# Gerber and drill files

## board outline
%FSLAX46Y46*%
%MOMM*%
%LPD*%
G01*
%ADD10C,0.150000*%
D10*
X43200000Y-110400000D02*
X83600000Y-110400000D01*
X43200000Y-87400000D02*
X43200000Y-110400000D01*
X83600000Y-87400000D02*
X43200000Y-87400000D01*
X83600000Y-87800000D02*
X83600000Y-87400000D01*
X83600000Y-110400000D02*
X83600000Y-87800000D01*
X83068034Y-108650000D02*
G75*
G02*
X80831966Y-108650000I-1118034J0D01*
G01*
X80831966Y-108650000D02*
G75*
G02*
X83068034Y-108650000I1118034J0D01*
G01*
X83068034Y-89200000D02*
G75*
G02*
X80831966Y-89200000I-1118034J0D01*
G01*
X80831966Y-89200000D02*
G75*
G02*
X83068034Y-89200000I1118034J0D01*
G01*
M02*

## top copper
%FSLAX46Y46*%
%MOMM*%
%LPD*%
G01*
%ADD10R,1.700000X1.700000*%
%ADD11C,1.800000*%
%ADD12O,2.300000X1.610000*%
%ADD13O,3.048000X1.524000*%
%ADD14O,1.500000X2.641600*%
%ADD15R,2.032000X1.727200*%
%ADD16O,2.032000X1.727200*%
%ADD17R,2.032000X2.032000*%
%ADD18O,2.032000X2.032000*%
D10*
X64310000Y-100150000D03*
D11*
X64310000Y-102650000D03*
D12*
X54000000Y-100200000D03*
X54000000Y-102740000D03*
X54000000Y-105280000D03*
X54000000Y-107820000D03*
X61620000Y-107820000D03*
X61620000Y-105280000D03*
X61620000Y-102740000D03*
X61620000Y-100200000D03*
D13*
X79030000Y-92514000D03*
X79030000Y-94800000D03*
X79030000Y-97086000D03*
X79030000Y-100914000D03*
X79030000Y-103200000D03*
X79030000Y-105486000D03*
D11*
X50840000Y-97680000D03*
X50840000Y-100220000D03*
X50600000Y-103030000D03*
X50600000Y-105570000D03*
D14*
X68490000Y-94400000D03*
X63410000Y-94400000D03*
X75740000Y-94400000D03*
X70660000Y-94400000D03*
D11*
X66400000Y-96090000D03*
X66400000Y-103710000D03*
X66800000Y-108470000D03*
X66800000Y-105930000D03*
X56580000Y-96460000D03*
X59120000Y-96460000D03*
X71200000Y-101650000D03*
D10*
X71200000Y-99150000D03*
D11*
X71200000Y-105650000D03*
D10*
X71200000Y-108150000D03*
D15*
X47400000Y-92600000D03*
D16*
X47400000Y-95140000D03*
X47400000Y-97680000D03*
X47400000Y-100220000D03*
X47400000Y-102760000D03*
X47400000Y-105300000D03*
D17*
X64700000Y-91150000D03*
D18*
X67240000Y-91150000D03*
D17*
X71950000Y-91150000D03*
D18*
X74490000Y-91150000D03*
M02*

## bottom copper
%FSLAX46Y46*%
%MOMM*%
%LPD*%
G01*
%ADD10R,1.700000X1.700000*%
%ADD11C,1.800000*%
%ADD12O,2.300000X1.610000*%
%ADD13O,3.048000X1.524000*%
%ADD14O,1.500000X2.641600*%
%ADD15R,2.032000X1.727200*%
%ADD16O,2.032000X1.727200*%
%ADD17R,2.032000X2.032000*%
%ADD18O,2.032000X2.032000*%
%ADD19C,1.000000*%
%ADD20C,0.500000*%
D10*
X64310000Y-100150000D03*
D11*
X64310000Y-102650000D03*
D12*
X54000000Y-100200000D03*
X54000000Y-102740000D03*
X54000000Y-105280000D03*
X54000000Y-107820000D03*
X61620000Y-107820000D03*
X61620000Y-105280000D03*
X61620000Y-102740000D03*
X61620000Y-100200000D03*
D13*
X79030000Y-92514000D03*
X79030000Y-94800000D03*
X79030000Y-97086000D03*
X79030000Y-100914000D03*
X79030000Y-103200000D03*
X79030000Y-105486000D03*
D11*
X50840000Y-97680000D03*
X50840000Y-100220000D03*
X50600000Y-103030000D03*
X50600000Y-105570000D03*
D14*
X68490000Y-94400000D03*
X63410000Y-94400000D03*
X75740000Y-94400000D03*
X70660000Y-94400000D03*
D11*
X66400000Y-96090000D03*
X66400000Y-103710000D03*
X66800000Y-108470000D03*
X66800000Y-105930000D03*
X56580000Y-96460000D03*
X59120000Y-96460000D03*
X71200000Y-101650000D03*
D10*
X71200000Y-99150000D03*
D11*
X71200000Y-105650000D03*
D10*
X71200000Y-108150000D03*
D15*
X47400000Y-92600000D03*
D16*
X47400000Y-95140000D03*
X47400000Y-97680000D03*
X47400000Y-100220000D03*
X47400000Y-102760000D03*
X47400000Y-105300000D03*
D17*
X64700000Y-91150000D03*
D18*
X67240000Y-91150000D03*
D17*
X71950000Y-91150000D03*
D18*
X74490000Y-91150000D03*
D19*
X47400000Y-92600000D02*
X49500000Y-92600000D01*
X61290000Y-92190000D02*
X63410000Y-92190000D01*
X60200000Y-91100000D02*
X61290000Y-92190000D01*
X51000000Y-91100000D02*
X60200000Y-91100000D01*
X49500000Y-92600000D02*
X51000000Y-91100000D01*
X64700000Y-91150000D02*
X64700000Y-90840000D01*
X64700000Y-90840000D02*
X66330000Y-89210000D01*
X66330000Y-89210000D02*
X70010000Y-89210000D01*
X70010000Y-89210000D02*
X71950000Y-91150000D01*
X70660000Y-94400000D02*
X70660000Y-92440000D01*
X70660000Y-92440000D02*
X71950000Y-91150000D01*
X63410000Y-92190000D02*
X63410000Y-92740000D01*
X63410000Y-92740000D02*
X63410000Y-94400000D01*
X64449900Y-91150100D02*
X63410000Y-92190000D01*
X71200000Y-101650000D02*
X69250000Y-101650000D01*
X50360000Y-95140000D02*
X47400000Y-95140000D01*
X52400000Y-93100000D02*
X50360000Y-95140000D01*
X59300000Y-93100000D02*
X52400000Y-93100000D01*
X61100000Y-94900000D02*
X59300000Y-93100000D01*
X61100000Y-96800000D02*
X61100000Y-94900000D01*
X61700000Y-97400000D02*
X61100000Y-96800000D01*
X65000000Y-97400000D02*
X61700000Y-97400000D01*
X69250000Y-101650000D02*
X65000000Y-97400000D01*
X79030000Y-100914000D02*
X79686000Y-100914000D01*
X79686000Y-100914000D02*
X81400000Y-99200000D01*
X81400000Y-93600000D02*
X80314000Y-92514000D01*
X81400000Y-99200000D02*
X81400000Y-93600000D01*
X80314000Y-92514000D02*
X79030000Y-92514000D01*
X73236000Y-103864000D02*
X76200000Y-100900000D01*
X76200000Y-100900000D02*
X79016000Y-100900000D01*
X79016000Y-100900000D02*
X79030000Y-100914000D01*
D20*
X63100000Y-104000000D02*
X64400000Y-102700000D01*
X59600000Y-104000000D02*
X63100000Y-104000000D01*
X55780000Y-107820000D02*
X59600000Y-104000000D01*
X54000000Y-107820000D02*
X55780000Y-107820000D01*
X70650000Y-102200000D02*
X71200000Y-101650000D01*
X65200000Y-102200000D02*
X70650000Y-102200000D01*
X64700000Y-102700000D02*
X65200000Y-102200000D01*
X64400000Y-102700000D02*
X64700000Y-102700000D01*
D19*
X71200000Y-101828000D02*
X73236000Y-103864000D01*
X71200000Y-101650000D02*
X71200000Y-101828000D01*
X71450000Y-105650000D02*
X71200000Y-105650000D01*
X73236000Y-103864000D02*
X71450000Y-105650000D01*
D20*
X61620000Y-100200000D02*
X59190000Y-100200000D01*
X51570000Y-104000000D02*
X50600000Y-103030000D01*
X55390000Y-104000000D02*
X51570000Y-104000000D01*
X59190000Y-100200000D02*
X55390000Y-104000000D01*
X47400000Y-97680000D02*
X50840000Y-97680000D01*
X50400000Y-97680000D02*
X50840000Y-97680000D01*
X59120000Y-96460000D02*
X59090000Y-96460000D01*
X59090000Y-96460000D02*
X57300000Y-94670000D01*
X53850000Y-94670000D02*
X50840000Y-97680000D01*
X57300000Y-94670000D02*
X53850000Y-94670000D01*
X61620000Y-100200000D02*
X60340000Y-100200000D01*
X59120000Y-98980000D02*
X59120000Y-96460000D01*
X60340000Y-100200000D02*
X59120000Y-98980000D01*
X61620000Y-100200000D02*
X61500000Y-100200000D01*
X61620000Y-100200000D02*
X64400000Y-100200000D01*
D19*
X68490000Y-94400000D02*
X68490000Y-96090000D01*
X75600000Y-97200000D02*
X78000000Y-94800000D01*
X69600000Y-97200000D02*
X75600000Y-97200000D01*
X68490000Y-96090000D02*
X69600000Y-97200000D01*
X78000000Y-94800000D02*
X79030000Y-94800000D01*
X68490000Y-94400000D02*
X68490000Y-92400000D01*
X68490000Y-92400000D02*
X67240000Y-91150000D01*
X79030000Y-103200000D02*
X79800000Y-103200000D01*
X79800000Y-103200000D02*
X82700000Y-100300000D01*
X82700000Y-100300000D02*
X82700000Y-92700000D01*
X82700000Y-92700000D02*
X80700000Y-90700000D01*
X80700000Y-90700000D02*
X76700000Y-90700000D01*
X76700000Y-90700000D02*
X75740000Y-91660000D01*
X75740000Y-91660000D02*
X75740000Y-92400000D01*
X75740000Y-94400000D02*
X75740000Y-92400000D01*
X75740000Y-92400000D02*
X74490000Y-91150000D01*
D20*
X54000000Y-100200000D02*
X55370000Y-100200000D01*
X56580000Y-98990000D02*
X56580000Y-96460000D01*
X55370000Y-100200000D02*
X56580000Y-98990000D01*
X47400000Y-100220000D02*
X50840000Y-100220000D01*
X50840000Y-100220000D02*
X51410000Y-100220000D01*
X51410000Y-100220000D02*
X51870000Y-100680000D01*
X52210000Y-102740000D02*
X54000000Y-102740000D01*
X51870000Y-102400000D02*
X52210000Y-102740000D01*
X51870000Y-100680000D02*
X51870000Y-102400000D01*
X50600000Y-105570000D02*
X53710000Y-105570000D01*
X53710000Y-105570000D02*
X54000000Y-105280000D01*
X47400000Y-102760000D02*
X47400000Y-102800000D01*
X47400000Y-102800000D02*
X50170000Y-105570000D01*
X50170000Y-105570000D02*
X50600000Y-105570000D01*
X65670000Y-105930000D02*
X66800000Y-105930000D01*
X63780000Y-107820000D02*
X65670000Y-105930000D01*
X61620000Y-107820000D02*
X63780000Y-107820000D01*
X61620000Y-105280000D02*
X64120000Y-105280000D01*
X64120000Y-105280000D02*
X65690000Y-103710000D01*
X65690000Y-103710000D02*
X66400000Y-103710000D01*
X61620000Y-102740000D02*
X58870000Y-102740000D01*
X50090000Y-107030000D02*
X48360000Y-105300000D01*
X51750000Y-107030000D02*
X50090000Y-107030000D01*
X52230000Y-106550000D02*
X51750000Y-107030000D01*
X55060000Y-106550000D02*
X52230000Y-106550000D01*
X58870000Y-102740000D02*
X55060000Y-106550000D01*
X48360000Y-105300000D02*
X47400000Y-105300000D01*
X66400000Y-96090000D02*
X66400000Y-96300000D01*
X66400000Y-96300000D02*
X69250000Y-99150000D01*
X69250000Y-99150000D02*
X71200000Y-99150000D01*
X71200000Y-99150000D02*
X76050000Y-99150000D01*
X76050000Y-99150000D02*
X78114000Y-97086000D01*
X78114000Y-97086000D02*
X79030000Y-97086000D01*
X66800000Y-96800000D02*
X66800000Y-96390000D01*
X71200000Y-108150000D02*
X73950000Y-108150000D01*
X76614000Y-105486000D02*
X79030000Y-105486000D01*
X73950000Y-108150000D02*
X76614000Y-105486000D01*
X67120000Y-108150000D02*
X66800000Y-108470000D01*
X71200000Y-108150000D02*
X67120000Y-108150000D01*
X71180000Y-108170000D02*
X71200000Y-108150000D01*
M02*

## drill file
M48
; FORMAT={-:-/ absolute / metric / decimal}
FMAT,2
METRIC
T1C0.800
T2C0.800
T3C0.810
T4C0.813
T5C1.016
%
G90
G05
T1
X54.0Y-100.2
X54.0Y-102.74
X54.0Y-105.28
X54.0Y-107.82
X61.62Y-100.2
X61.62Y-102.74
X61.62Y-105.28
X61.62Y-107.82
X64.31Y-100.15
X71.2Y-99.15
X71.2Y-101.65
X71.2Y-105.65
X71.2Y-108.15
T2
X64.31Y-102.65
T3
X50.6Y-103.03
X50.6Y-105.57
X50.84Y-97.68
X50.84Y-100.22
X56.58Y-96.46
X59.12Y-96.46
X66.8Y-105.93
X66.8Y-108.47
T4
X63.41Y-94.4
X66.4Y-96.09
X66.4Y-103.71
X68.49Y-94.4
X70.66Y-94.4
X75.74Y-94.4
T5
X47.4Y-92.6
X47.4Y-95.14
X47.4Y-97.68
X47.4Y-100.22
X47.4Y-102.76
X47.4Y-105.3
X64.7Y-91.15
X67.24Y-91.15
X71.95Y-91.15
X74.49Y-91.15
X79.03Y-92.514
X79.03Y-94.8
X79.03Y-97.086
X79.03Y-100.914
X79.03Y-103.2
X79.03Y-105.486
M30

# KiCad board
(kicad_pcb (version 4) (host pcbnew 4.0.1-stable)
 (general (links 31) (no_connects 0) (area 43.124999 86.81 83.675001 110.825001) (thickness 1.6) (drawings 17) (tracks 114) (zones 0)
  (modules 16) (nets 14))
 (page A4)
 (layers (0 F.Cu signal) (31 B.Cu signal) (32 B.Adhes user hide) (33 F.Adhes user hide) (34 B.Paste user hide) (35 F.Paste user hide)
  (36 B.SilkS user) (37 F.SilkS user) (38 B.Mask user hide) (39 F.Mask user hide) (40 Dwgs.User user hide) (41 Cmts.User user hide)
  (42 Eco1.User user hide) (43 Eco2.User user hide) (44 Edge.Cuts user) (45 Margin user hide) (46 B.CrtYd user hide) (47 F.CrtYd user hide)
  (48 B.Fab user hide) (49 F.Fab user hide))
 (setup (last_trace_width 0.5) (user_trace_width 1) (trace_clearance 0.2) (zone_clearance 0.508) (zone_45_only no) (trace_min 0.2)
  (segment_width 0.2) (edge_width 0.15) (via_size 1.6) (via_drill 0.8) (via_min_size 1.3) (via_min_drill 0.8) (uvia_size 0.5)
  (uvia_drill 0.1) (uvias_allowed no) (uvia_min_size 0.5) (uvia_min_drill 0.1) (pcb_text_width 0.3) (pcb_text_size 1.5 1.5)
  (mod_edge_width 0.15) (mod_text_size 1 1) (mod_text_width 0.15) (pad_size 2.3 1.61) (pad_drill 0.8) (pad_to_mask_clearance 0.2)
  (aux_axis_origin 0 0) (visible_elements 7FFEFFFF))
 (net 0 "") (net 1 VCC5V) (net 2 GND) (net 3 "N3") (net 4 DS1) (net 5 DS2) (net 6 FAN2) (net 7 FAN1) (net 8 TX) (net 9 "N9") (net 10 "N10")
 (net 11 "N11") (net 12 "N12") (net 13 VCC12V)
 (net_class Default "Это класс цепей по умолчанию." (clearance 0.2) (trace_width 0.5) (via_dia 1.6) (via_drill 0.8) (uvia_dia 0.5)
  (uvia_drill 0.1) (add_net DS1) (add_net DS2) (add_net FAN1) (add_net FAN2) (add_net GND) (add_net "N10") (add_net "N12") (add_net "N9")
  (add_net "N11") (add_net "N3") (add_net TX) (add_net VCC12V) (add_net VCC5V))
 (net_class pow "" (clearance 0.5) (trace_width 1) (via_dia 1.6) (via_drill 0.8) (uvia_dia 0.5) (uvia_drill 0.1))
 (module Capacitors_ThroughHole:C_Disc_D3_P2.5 (layer F.Cu) (at 64.31 100.15 270)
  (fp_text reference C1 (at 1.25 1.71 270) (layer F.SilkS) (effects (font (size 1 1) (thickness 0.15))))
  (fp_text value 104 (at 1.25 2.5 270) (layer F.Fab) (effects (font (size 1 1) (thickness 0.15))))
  (pad 1 thru_hole rect (at 0 0 270) (size 1.7 1.7) (drill 0.8) (layers *.Cu *.Mask F.SilkS) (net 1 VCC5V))
  (pad 2 thru_hole circle (at 2.5 0 270) (size 1.8 1.8) (drill 0.8001) (layers *.Cu *.Mask F.SilkS) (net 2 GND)))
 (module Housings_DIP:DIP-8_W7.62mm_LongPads (layer F.Cu) (at 54 100.2)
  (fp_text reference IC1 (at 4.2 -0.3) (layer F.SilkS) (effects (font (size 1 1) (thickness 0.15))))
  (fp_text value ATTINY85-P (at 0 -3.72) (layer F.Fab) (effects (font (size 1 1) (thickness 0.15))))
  (pad 1 thru_hole oval (at 0 0) (size 2.3 1.61) (drill 0.8) (layers *.Cu *.Mask F.SilkS) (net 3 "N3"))
  (pad 2 thru_hole oval (at 0 2.54) (size 2.3 1.61) (drill 0.8) (layers *.Cu *.Mask F.SilkS) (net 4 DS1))
  (pad 3 thru_hole oval (at 0 5.08) (size 2.3 1.61) (drill 0.8) (layers *.Cu *.Mask F.SilkS) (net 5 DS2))
  (pad 4 thru_hole oval (at 0 7.62) (size 2.3 1.61) (drill 0.8) (layers *.Cu *.Mask F.SilkS) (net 2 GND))
  (pad 5 thru_hole oval (at 7.62 7.62) (size 2.3 1.61) (drill 0.8) (layers *.Cu *.Mask F.SilkS) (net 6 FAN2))
  (pad 6 thru_hole oval (at 7.62 5.08) (size 2.3 1.61) (drill 0.8) (layers *.Cu *.Mask F.SilkS) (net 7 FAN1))
  (pad 7 thru_hole oval (at 7.62 2.54) (size 2.3 1.61) (drill 0.8) (layers *.Cu *.Mask F.SilkS) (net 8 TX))
  (pad 8 thru_hole oval (at 7.62 0) (size 2.3 1.61) (drill 0.8) (layers *.Cu *.Mask F.SilkS) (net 1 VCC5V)))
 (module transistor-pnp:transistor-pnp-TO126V (layer F.Cu) (at 80.3 94.8 270)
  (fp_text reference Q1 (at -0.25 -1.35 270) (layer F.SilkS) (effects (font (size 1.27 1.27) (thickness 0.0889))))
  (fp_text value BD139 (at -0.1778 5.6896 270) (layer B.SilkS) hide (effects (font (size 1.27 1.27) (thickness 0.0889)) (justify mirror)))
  (pad 1 thru_hole oval (at -2.286 1.27 270) (size 1.524 3.048) (drill 1.016) (layers *.Cu F.Paste F.SilkS F.Mask) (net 2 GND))
  (pad 2 thru_hole oval (at 0 1.27 270) (size 1.524 3.048) (drill 1.016) (layers *.Cu F.Paste F.SilkS F.Mask) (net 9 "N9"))
  (pad 3 thru_hole oval (at 2.286 1.27 270) (size 1.524 3.048) (drill 1.016) (layers *.Cu F.Paste F.SilkS F.Mask) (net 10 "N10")))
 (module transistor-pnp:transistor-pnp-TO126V (layer F.Cu) (at 80.3 103.2 270)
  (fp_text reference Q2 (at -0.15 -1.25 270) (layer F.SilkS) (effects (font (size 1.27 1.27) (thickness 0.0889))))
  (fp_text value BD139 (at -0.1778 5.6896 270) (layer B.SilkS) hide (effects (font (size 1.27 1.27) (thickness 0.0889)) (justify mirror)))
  (pad 1 thru_hole oval (at -2.286 1.27 270) (size 1.524 3.048) (drill 1.016) (layers *.Cu F.Paste F.SilkS F.Mask) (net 2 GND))
  (pad 2 thru_hole oval (at 0 1.27 270) (size 1.524 3.048) (drill 1.016) (layers *.Cu F.Paste F.SilkS F.Mask) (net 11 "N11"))
  (pad 3 thru_hole oval (at 2.286 1.27 270) (size 1.524 3.048) (drill 1.016) (layers *.Cu F.Paste F.SilkS F.Mask) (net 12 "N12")))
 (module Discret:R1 (layer F.Cu) (at 50.84 98.95 270)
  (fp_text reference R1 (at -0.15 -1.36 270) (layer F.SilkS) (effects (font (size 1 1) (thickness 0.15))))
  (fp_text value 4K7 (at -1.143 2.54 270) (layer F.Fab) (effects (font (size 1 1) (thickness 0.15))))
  (pad 1 thru_hole circle (at -1.27 0 270) (size 1.8 1.8) (drill 0.81) (layers *.Cu *.Mask F.SilkS) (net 1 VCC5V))
  (pad 2 thru_hole circle (at 1.27 0 270) (size 1.8 1.8) (drill 0.81) (layers *.Cu *.Mask F.SilkS) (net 4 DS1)))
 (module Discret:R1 (layer F.Cu) (at 50.6 104.3 270)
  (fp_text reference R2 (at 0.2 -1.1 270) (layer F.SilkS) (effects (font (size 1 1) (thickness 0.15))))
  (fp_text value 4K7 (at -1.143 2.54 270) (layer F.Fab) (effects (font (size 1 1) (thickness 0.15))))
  (pad 1 thru_hole circle (at -1.27 0 270) (size 1.8 1.8) (drill 0.81) (layers *.Cu *.Mask F.SilkS) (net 1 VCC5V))
  (pad 2 thru_hole circle (at 1.27 0 270) (size 1.8 1.8) (drill 0.81) (layers *.Cu *.Mask F.SilkS) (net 5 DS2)))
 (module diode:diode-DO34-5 (layer F.Cu) (at 65.95 94.4)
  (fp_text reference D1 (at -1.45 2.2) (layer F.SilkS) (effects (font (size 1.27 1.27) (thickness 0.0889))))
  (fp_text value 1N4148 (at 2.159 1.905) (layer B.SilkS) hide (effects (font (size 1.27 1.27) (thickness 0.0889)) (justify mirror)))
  (pad 2 thru_hole oval (at 2.54 0) (size 1.5 2.6416) (drill 0.8128) (layers *.Cu F.Paste F.SilkS F.Mask) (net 9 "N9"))
  (pad 1 thru_hole oval (at -2.54 0) (size 1.5 2.6416) (drill 0.8128) (layers *.Cu F.Paste F.SilkS F.Mask) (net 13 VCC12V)))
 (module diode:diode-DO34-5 (layer F.Cu) (at 73.2 94.4)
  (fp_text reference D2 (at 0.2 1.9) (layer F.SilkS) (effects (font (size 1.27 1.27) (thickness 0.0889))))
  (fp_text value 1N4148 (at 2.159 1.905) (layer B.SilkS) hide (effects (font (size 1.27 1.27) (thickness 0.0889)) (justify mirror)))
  (pad 2 thru_hole oval (at 2.54 0) (size 1.5 2.6416) (drill 0.8128) (layers *.Cu F.Paste F.SilkS F.Mask) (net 11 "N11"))
  (pad 1 thru_hole oval (at -2.54 0) (size 1.5 2.6416) (drill 0.8128) (layers *.Cu F.Paste F.SilkS F.Mask) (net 13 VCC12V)))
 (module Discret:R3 (layer F.Cu) (at 66.4 99.9 270)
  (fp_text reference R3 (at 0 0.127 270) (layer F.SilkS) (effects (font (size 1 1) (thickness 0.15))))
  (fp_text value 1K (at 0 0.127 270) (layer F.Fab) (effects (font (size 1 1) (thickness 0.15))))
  (pad 1 thru_hole circle (at -3.81 0 270) (size 1.8 1.8) (drill 0.8128) (layers *.Cu *.Mask F.SilkS) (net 10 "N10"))
  (pad 2 thru_hole circle (at 3.81 0 270) (size 1.8 1.8) (drill 0.8128) (layers *.Cu *.Mask F.SilkS) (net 7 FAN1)))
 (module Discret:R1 (layer F.Cu) (at 66.8 107.2 90)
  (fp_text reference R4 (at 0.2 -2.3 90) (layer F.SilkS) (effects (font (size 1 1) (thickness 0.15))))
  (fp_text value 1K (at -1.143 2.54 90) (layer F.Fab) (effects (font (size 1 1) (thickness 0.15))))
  (pad 1 thru_hole circle (at -1.27 0 90) (size 1.8 1.8) (drill 0.81) (layers *.Cu *.Mask F.SilkS) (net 12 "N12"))
  (pad 2 thru_hole circle (at 1.27 0 90) (size 1.8 1.8) (drill 0.81) (layers *.Cu *.Mask F.SilkS) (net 6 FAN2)))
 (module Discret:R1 (layer F.Cu) (at 57.85 96.46)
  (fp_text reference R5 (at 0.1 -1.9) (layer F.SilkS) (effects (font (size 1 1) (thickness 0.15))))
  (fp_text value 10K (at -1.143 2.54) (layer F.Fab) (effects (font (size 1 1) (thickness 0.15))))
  (pad 1 thru_hole circle (at -1.27 0) (size 1.8 1.8) (drill 0.81) (layers *.Cu *.Mask F.SilkS) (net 3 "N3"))
  (pad 2 thru_hole circle (at 1.27 0) (size 1.8 1.8) (drill 0.81) (layers *.Cu *.Mask F.SilkS) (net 1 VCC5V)))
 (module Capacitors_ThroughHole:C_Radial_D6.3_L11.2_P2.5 (layer F.Cu) (at 71.2 99.15 270)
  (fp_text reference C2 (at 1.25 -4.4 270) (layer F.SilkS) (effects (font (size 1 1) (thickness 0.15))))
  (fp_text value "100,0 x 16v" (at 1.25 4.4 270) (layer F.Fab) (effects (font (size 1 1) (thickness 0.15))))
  (pad 2 thru_hole circle (at 2.5 0 270) (size 1.8 1.8) (drill 0.8) (layers *.Cu *.Mask F.SilkS) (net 2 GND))
  (pad 1 thru_hole rect (at 0 0 270) (size 1.7 1.7) (drill 0.8) (layers *.Cu *.Mask F.SilkS) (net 10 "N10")))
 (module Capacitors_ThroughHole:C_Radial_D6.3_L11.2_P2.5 (layer F.Cu) (at 71.2 108.15 90)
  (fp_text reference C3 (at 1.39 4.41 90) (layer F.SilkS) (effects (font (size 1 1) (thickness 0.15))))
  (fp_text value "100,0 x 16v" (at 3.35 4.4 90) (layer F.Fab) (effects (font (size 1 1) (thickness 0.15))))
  (pad 2 thru_hole circle (at 2.5 0 90) (size 1.8 1.8) (drill 0.8) (layers *.Cu *.Mask F.SilkS) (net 2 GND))
  (pad 1 thru_hole rect (at 0 0 90) (size 1.7 1.7) (drill 0.8) (layers *.Cu *.Mask F.SilkS) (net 12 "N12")))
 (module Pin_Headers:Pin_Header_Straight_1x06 (layer F.Cu) (at 47.4 92.6)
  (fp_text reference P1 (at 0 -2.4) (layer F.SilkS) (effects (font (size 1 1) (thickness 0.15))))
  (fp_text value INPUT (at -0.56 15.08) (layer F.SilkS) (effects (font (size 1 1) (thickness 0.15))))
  (pad 1 thru_hole rect (at 0 0) (size 2.032 1.7272) (drill 1.016) (layers *.Cu *.Mask F.SilkS) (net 13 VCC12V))
  (pad 2 thru_hole oval (at 0 2.54) (size 2.032 1.7272) (drill 1.016) (layers *.Cu *.Mask F.SilkS) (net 2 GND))
  (pad 3 thru_hole oval (at 0 5.08) (size 2.032 1.7272) (drill 1.016) (layers *.Cu *.Mask F.SilkS) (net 1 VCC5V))
  (pad 4 thru_hole oval (at 0 7.62) (size 2.032 1.7272) (drill 1.016) (layers *.Cu *.Mask F.SilkS) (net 4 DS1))
  (pad 5 thru_hole oval (at 0 10.16) (size 2.032 1.7272) (drill 1.016) (layers *.Cu *.Mask F.SilkS) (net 5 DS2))
  (pad 6 thru_hole oval (at 0 12.7) (size 2.032 1.7272) (drill 1.016) (layers *.Cu *.Mask F.SilkS) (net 8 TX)))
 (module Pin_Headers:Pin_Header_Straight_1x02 (layer F.Cu) (at 64.7 91.15 90)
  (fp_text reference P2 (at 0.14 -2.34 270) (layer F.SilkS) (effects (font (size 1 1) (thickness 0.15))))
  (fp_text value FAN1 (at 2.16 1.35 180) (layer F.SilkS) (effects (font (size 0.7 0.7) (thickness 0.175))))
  (pad 1 thru_hole rect (at 0 0 90) (size 2.032 2.032) (drill 1.016) (layers *.Cu *.Mask F.SilkS) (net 13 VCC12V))
  (pad 2 thru_hole oval (at 0 2.54 90) (size 2.032 2.032) (drill 1.016) (layers *.Cu *.Mask F.SilkS) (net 9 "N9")))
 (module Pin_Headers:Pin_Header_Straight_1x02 (layer F.Cu) (at 71.95 91.15 90)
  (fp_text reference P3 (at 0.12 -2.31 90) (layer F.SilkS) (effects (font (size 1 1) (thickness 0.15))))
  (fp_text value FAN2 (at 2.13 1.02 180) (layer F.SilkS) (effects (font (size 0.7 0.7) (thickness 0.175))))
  (pad 1 thru_hole rect (at 0 0 90) (size 2.032 2.032) (drill 1.016) (layers *.Cu *.Mask F.SilkS) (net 13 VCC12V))
  (pad 2 thru_hole oval (at 0 2.54 90) (size 2.032 2.032) (drill 1.016) (layers *.Cu *.Mask F.SilkS) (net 11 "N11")))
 (gr_line (start 43.2 110.4) (end 83.6 110.4) (angle 90) (layer Edge.Cuts) (width 0.15))
 (gr_line (start 43.2 87.4) (end 43.2 110.4) (angle 90) (layer Edge.Cuts) (width 0.15))
 (gr_line (start 83.6 87.4) (end 43.2 87.4) (angle 90) (layer Edge.Cuts) (width 0.15))
 (gr_line (start 83.6 87.8) (end 83.6 87.4) (angle 90) (layer Edge.Cuts) (width 0.15))
 (gr_line (start 83.6 110.4) (end 83.6 87.8) (angle 90) (layer Edge.Cuts) (width 0.15))
 (gr_circle (center 81.95 108.65) (end 82.95 108.15) (layer Edge.Cuts) (width 0.15))
 (gr_circle (center 81.95 89.2) (end 82.95 88.7) (layer Edge.Cuts) (width 0.15))
 (segment (start 47.4 92.6) (end 49.5 92.6) (width 1) (layer B.Cu) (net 13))
 (segment (start 61.29 92.19) (end 63.41 92.19) (width 1) (layer B.Cu) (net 13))
 (segment (start 60.2 91.1) (end 61.29 92.19) (width 1) (layer B.Cu) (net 13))
 (segment (start 51 91.1) (end 60.2 91.1) (width 1) (layer B.Cu) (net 13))
 (segment (start 49.5 92.6) (end 51 91.1) (width 1) (layer B.Cu) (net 13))
 (segment (start 64.7 91.15) (end 64.7 90.84) (width 1) (layer B.Cu) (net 13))
 (segment (start 64.7 90.84) (end 66.33 89.21) (width 1) (layer B.Cu) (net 13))
 (segment (start 66.33 89.21) (end 70.01 89.21) (width 1) (layer B.Cu) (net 13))
 (segment (start 70.01 89.21) (end 71.95 91.15) (width 1) (layer B.Cu) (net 13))
 (segment (start 70.66 94.4) (end 70.66 92.44) (width 1) (layer B.Cu) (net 13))
 (segment (start 70.66 92.44) (end 71.95 91.15) (width 1) (layer B.Cu) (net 13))
 (segment (start 63.41 92.19) (end 63.41 92.74) (width 1) (layer B.Cu) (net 13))
 (segment (start 63.41 92.74) (end 63.41 94.4) (width 1) (layer B.Cu) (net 13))
 (segment (start 64.4499 91.1501) (end 63.41 92.19) (width 1) (layer B.Cu) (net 13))
 (segment (start 71.2 101.65) (end 69.25 101.65) (width 1) (layer B.Cu) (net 2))
 (segment (start 50.36 95.14) (end 47.4 95.14) (width 1) (layer B.Cu) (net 2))
 (segment (start 52.4 93.1) (end 50.36 95.14) (width 1) (layer B.Cu) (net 2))
 (segment (start 59.3 93.1) (end 52.4 93.1) (width 1) (layer B.Cu) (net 2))
 (segment (start 61.1 94.9) (end 59.3 93.1) (width 1) (layer B.Cu) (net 2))
 (segment (start 61.1 96.8) (end 61.1 94.9) (width 1) (layer B.Cu) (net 2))
 (segment (start 61.7 97.4) (end 61.1 96.8) (width 1) (layer B.Cu) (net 2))
 (segment (start 65 97.4) (end 61.7 97.4) (width 1) (layer B.Cu) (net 2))
 (segment (start 69.25 101.65) (end 65 97.4) (width 1) (layer B.Cu) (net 2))
 (segment (start 79.03 100.914) (end 79.686 100.914) (width 1) (layer B.Cu) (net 2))
 (segment (start 79.686 100.914) (end 81.4 99.2) (width 1) (layer B.Cu) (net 2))
 (segment (start 81.4 93.6) (end 80.314 92.514) (width 1) (layer B.Cu) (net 2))
 (segment (start 81.4 99.2) (end 81.4 93.6) (width 1) (layer B.Cu) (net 2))
 (segment (start 80.314 92.514) (end 79.03 92.514) (width 1) (layer B.Cu) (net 2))
 (segment (start 73.236 103.864) (end 76.2 100.9) (width 1) (layer B.Cu) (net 2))
 (segment (start 76.2 100.9) (end 79.016 100.9) (width 1) (layer B.Cu) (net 2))
 (segment (start 79.016 100.9) (end 79.03 100.914) (width 1) (layer B.Cu) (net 2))
 (segment (start 63.1 104) (end 64.4 102.7) (width 0.5) (layer B.Cu) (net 2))
 (segment (start 59.6 104) (end 63.1 104) (width 0.5) (layer B.Cu) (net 2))
 (segment (start 55.78 107.82) (end 59.6 104) (width 0.5) (layer B.Cu) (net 2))
 (segment (start 54 107.82) (end 55.78 107.82) (width 0.5) (layer B.Cu) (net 2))
 (segment (start 70.65 102.2) (end 71.2 101.65) (width 0.5) (layer B.Cu) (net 2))
 (segment (start 65.2 102.2) (end 70.65 102.2) (width 0.5) (layer B.Cu) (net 2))
 (segment (start 64.7 102.7) (end 65.2 102.2) (width 0.5) (layer B.Cu) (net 2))
 (segment (start 64.4 102.7) (end 64.7 102.7) (width 0.5) (layer B.Cu) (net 2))
 (segment (start 71.2 101.828) (end 73.236 103.864) (width 1) (layer B.Cu) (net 2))
 (segment (start 71.2 101.65) (end 71.2 101.828) (width 1) (layer B.Cu) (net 2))
 (segment (start 71.45 105.65) (end 71.2 105.65) (width 1) (layer B.Cu) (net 2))
 (segment (start 73.236 103.864) (end 71.45 105.65) (width 1) (layer B.Cu) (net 2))
 (segment (start 61.62 100.2) (end 59.19 100.2) (width 0.5) (layer B.Cu) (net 1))
 (segment (start 51.57 104) (end 50.6 103.03) (width 0.5) (layer B.Cu) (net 1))
 (segment (start 55.39 104) (end 51.57 104) (width 0.5) (layer B.Cu) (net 1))
 (segment (start 59.19 100.2) (end 55.39 104) (width 0.5) (layer B.Cu) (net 1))
 (segment (start 47.4 97.68) (end 50.84 97.68) (width 0.5) (layer B.Cu) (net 1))
 (segment (start 50.4 97.68) (end 50.84 97.68) (width 0.5) (layer B.Cu) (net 1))
 (segment (start 59.12 96.46) (end 59.09 96.46) (width 0.5) (layer B.Cu) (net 1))
 (segment (start 59.09 96.46) (end 57.3 94.67) (width 0.5) (layer B.Cu) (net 1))
 (segment (start 53.85 94.67) (end 50.84 97.68) (width 0.5) (layer B.Cu) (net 1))
 (segment (start 57.3 94.67) (end 53.85 94.67) (width 0.5) (layer B.Cu) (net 1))
 (segment (start 61.62 100.2) (end 60.34 100.2) (width 0.5) (layer B.Cu) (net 1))
 (segment (start 59.12 98.98) (end 59.12 96.46) (width 0.5) (layer B.Cu) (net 1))
 (segment (start 60.34 100.2) (end 59.12 98.98) (width 0.5) (layer B.Cu) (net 1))
 (segment (start 61.62 100.2) (end 61.5 100.2) (width 0.5) (layer B.Cu) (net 1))
 (segment (start 61.62 100.2) (end 64.4 100.2) (width 0.5) (layer B.Cu) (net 1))
 (segment (start 68.49 94.4) (end 68.49 96.09) (width 1) (layer B.Cu) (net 9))
 (segment (start 75.6 97.2) (end 78 94.8) (width 1) (layer B.Cu) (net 9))
 (segment (start 69.6 97.2) (end 75.6 97.2) (width 1) (layer B.Cu) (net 9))
 (segment (start 68.49 96.09) (end 69.6 97.2) (width 1) (layer B.Cu) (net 9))
 (segment (start 78 94.8) (end 79.03 94.8) (width 1) (layer B.Cu) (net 9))
 (segment (start 68.49 94.4) (end 68.49 92.4) (width 1) (layer B.Cu) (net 9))
 (segment (start 68.49 92.4) (end 67.24 91.15) (width 1) (layer B.Cu) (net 9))
 (segment (start 79.03 103.2) (end 79.8 103.2) (width 1) (layer B.Cu) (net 11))
 (segment (start 79.8 103.2) (end 82.7 100.3) (width 1) (layer B.Cu) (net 11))
 (segment (start 82.7 100.3) (end 82.7 92.7) (width 1) (layer B.Cu) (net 11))
 (segment (start 82.7 92.7) (end 80.7 90.7) (width 1) (layer B.Cu) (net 11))
 (segment (start 80.7 90.7) (end 76.7 90.7) (width 1) (layer B.Cu) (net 11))
 (segment (start 76.7 90.7) (end 75.74 91.66) (width 1) (layer B.Cu) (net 11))
 (segment (start 75.74 91.66) (end 75.74 92.4) (width 1) (layer B.Cu) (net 11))
 (segment (start 75.74 94.4) (end 75.74 92.4) (width 1) (layer B.Cu) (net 11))
 (segment (start 75.74 92.4) (end 74.49 91.15) (width 1) (layer B.Cu) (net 11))
 (segment (start 54 100.2) (end 55.37 100.2) (width 0.5) (layer B.Cu) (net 3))
 (segment (start 56.58 98.99) (end 56.58 96.46) (width 0.5) (layer B.Cu) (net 3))
 (segment (start 55.37 100.2) (end 56.58 98.99) (width 0.5) (layer B.Cu) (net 3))
 (segment (start 47.4 100.22) (end 50.84 100.22) (width 0.5) (layer B.Cu) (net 4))
 (segment (start 50.84 100.22) (end 51.41 100.22) (width 0.5) (layer B.Cu) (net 4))
 (segment (start 51.41 100.22) (end 51.87 100.68) (width 0.5) (layer B.Cu) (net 4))
 (segment (start 52.21 102.74) (end 54 102.74) (width 0.5) (layer B.Cu) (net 4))
 (segment (start 51.87 102.4) (end 52.21 102.74) (width 0.5) (layer B.Cu) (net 4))
 (segment (start 51.87 100.68) (end 51.87 102.4) (width 0.5) (layer B.Cu) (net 4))
 (segment (start 50.6 105.57) (end 53.71 105.57) (width 0.5) (layer B.Cu) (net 5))
 (segment (start 53.71 105.57) (end 54 105.28) (width 0.5) (layer B.Cu) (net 5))
 (segment (start 47.4 102.76) (end 47.4 102.8) (width 0.5) (layer B.Cu) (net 5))
 (segment (start 47.4 102.8) (end 50.17 105.57) (width 0.5) (layer B.Cu) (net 5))
 (segment (start 50.17 105.57) (end 50.6 105.57) (width 0.5) (layer B.Cu) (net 5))
 (segment (start 65.67 105.93) (end 66.8 105.93) (width 0.5) (layer B.Cu) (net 6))
 (segment (start 63.78 107.82) (end 65.67 105.93) (width 0.5) (layer B.Cu) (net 6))
 (segment (start 61.62 107.82) (end 63.78 107.82) (width 0.5) (layer B.Cu) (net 6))
 (segment (start 61.62 105.28) (end 64.12 105.28) (width 0.5) (layer B.Cu) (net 7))
 (segment (start 64.12 105.28) (end 65.69 103.71) (width 0.5) (layer B.Cu) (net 7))
 (segment (start 65.69 103.71) (end 66.4 103.71) (width 0.5) (layer B.Cu) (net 7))
 (segment (start 61.62 102.74) (end 58.87 102.74) (width 0.5) (layer B.Cu) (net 8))
 (segment (start 50.09 107.03) (end 48.36 105.3) (width 0.5) (layer B.Cu) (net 8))
 (segment (start 51.75 107.03) (end 50.09 107.03) (width 0.5) (layer B.Cu) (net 8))
 (segment (start 52.23 106.55) (end 51.75 107.03) (width 0.5) (layer B.Cu) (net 8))
 (segment (start 55.06 106.55) (end 52.23 106.55) (width 0.5) (layer B.Cu) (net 8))
 (segment (start 58.87 102.74) (end 55.06 106.55) (width 0.5) (layer B.Cu) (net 8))
 (segment (start 48.36 105.3) (end 47.4 105.3) (width 0.5) (layer B.Cu) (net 8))
 (segment (start 66.4 96.09) (end 66.4 96.3) (width 0.5) (layer B.Cu) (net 10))
 (segment (start 66.4 96.3) (end 69.25 99.15) (width 0.5) (layer B.Cu) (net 10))
 (segment (start 69.25 99.15) (end 71.2 99.15) (width 0.5) (layer B.Cu) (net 10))
 (segment (start 71.2 99.15) (end 76.05 99.15) (width 0.5) (layer B.Cu) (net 10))
 (segment (start 76.05 99.15) (end 78.114 97.086) (width 0.5) (layer B.Cu) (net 10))
 (segment (start 78.114 97.086) (end 79.03 97.086) (width 0.5) (layer B.Cu) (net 10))
 (segment (start 66.8 96.8) (end 66.8 96.39) (width 0.5) (layer B.Cu) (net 10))
 (segment (start 71.2 108.15) (end 73.95 108.15) (width 0.5) (layer B.Cu) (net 12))
 (segment (start 76.614 105.486) (end 79.03 105.486) (width 0.5) (layer B.Cu) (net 12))
 (segment (start 73.95 108.15) (end 76.614 105.486) (width 0.5) (layer B.Cu) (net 12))
 (segment (start 67.12 108.15) (end 66.8 108.47) (width 0.5) (layer B.Cu) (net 12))
 (segment (start 71.2 108.15) (end 67.12 108.15) (width 0.5) (layer B.Cu) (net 12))
 (segment (start 71.18 108.17) (end 71.2 108.15) (width 0.5) (layer B.Cu) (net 12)))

